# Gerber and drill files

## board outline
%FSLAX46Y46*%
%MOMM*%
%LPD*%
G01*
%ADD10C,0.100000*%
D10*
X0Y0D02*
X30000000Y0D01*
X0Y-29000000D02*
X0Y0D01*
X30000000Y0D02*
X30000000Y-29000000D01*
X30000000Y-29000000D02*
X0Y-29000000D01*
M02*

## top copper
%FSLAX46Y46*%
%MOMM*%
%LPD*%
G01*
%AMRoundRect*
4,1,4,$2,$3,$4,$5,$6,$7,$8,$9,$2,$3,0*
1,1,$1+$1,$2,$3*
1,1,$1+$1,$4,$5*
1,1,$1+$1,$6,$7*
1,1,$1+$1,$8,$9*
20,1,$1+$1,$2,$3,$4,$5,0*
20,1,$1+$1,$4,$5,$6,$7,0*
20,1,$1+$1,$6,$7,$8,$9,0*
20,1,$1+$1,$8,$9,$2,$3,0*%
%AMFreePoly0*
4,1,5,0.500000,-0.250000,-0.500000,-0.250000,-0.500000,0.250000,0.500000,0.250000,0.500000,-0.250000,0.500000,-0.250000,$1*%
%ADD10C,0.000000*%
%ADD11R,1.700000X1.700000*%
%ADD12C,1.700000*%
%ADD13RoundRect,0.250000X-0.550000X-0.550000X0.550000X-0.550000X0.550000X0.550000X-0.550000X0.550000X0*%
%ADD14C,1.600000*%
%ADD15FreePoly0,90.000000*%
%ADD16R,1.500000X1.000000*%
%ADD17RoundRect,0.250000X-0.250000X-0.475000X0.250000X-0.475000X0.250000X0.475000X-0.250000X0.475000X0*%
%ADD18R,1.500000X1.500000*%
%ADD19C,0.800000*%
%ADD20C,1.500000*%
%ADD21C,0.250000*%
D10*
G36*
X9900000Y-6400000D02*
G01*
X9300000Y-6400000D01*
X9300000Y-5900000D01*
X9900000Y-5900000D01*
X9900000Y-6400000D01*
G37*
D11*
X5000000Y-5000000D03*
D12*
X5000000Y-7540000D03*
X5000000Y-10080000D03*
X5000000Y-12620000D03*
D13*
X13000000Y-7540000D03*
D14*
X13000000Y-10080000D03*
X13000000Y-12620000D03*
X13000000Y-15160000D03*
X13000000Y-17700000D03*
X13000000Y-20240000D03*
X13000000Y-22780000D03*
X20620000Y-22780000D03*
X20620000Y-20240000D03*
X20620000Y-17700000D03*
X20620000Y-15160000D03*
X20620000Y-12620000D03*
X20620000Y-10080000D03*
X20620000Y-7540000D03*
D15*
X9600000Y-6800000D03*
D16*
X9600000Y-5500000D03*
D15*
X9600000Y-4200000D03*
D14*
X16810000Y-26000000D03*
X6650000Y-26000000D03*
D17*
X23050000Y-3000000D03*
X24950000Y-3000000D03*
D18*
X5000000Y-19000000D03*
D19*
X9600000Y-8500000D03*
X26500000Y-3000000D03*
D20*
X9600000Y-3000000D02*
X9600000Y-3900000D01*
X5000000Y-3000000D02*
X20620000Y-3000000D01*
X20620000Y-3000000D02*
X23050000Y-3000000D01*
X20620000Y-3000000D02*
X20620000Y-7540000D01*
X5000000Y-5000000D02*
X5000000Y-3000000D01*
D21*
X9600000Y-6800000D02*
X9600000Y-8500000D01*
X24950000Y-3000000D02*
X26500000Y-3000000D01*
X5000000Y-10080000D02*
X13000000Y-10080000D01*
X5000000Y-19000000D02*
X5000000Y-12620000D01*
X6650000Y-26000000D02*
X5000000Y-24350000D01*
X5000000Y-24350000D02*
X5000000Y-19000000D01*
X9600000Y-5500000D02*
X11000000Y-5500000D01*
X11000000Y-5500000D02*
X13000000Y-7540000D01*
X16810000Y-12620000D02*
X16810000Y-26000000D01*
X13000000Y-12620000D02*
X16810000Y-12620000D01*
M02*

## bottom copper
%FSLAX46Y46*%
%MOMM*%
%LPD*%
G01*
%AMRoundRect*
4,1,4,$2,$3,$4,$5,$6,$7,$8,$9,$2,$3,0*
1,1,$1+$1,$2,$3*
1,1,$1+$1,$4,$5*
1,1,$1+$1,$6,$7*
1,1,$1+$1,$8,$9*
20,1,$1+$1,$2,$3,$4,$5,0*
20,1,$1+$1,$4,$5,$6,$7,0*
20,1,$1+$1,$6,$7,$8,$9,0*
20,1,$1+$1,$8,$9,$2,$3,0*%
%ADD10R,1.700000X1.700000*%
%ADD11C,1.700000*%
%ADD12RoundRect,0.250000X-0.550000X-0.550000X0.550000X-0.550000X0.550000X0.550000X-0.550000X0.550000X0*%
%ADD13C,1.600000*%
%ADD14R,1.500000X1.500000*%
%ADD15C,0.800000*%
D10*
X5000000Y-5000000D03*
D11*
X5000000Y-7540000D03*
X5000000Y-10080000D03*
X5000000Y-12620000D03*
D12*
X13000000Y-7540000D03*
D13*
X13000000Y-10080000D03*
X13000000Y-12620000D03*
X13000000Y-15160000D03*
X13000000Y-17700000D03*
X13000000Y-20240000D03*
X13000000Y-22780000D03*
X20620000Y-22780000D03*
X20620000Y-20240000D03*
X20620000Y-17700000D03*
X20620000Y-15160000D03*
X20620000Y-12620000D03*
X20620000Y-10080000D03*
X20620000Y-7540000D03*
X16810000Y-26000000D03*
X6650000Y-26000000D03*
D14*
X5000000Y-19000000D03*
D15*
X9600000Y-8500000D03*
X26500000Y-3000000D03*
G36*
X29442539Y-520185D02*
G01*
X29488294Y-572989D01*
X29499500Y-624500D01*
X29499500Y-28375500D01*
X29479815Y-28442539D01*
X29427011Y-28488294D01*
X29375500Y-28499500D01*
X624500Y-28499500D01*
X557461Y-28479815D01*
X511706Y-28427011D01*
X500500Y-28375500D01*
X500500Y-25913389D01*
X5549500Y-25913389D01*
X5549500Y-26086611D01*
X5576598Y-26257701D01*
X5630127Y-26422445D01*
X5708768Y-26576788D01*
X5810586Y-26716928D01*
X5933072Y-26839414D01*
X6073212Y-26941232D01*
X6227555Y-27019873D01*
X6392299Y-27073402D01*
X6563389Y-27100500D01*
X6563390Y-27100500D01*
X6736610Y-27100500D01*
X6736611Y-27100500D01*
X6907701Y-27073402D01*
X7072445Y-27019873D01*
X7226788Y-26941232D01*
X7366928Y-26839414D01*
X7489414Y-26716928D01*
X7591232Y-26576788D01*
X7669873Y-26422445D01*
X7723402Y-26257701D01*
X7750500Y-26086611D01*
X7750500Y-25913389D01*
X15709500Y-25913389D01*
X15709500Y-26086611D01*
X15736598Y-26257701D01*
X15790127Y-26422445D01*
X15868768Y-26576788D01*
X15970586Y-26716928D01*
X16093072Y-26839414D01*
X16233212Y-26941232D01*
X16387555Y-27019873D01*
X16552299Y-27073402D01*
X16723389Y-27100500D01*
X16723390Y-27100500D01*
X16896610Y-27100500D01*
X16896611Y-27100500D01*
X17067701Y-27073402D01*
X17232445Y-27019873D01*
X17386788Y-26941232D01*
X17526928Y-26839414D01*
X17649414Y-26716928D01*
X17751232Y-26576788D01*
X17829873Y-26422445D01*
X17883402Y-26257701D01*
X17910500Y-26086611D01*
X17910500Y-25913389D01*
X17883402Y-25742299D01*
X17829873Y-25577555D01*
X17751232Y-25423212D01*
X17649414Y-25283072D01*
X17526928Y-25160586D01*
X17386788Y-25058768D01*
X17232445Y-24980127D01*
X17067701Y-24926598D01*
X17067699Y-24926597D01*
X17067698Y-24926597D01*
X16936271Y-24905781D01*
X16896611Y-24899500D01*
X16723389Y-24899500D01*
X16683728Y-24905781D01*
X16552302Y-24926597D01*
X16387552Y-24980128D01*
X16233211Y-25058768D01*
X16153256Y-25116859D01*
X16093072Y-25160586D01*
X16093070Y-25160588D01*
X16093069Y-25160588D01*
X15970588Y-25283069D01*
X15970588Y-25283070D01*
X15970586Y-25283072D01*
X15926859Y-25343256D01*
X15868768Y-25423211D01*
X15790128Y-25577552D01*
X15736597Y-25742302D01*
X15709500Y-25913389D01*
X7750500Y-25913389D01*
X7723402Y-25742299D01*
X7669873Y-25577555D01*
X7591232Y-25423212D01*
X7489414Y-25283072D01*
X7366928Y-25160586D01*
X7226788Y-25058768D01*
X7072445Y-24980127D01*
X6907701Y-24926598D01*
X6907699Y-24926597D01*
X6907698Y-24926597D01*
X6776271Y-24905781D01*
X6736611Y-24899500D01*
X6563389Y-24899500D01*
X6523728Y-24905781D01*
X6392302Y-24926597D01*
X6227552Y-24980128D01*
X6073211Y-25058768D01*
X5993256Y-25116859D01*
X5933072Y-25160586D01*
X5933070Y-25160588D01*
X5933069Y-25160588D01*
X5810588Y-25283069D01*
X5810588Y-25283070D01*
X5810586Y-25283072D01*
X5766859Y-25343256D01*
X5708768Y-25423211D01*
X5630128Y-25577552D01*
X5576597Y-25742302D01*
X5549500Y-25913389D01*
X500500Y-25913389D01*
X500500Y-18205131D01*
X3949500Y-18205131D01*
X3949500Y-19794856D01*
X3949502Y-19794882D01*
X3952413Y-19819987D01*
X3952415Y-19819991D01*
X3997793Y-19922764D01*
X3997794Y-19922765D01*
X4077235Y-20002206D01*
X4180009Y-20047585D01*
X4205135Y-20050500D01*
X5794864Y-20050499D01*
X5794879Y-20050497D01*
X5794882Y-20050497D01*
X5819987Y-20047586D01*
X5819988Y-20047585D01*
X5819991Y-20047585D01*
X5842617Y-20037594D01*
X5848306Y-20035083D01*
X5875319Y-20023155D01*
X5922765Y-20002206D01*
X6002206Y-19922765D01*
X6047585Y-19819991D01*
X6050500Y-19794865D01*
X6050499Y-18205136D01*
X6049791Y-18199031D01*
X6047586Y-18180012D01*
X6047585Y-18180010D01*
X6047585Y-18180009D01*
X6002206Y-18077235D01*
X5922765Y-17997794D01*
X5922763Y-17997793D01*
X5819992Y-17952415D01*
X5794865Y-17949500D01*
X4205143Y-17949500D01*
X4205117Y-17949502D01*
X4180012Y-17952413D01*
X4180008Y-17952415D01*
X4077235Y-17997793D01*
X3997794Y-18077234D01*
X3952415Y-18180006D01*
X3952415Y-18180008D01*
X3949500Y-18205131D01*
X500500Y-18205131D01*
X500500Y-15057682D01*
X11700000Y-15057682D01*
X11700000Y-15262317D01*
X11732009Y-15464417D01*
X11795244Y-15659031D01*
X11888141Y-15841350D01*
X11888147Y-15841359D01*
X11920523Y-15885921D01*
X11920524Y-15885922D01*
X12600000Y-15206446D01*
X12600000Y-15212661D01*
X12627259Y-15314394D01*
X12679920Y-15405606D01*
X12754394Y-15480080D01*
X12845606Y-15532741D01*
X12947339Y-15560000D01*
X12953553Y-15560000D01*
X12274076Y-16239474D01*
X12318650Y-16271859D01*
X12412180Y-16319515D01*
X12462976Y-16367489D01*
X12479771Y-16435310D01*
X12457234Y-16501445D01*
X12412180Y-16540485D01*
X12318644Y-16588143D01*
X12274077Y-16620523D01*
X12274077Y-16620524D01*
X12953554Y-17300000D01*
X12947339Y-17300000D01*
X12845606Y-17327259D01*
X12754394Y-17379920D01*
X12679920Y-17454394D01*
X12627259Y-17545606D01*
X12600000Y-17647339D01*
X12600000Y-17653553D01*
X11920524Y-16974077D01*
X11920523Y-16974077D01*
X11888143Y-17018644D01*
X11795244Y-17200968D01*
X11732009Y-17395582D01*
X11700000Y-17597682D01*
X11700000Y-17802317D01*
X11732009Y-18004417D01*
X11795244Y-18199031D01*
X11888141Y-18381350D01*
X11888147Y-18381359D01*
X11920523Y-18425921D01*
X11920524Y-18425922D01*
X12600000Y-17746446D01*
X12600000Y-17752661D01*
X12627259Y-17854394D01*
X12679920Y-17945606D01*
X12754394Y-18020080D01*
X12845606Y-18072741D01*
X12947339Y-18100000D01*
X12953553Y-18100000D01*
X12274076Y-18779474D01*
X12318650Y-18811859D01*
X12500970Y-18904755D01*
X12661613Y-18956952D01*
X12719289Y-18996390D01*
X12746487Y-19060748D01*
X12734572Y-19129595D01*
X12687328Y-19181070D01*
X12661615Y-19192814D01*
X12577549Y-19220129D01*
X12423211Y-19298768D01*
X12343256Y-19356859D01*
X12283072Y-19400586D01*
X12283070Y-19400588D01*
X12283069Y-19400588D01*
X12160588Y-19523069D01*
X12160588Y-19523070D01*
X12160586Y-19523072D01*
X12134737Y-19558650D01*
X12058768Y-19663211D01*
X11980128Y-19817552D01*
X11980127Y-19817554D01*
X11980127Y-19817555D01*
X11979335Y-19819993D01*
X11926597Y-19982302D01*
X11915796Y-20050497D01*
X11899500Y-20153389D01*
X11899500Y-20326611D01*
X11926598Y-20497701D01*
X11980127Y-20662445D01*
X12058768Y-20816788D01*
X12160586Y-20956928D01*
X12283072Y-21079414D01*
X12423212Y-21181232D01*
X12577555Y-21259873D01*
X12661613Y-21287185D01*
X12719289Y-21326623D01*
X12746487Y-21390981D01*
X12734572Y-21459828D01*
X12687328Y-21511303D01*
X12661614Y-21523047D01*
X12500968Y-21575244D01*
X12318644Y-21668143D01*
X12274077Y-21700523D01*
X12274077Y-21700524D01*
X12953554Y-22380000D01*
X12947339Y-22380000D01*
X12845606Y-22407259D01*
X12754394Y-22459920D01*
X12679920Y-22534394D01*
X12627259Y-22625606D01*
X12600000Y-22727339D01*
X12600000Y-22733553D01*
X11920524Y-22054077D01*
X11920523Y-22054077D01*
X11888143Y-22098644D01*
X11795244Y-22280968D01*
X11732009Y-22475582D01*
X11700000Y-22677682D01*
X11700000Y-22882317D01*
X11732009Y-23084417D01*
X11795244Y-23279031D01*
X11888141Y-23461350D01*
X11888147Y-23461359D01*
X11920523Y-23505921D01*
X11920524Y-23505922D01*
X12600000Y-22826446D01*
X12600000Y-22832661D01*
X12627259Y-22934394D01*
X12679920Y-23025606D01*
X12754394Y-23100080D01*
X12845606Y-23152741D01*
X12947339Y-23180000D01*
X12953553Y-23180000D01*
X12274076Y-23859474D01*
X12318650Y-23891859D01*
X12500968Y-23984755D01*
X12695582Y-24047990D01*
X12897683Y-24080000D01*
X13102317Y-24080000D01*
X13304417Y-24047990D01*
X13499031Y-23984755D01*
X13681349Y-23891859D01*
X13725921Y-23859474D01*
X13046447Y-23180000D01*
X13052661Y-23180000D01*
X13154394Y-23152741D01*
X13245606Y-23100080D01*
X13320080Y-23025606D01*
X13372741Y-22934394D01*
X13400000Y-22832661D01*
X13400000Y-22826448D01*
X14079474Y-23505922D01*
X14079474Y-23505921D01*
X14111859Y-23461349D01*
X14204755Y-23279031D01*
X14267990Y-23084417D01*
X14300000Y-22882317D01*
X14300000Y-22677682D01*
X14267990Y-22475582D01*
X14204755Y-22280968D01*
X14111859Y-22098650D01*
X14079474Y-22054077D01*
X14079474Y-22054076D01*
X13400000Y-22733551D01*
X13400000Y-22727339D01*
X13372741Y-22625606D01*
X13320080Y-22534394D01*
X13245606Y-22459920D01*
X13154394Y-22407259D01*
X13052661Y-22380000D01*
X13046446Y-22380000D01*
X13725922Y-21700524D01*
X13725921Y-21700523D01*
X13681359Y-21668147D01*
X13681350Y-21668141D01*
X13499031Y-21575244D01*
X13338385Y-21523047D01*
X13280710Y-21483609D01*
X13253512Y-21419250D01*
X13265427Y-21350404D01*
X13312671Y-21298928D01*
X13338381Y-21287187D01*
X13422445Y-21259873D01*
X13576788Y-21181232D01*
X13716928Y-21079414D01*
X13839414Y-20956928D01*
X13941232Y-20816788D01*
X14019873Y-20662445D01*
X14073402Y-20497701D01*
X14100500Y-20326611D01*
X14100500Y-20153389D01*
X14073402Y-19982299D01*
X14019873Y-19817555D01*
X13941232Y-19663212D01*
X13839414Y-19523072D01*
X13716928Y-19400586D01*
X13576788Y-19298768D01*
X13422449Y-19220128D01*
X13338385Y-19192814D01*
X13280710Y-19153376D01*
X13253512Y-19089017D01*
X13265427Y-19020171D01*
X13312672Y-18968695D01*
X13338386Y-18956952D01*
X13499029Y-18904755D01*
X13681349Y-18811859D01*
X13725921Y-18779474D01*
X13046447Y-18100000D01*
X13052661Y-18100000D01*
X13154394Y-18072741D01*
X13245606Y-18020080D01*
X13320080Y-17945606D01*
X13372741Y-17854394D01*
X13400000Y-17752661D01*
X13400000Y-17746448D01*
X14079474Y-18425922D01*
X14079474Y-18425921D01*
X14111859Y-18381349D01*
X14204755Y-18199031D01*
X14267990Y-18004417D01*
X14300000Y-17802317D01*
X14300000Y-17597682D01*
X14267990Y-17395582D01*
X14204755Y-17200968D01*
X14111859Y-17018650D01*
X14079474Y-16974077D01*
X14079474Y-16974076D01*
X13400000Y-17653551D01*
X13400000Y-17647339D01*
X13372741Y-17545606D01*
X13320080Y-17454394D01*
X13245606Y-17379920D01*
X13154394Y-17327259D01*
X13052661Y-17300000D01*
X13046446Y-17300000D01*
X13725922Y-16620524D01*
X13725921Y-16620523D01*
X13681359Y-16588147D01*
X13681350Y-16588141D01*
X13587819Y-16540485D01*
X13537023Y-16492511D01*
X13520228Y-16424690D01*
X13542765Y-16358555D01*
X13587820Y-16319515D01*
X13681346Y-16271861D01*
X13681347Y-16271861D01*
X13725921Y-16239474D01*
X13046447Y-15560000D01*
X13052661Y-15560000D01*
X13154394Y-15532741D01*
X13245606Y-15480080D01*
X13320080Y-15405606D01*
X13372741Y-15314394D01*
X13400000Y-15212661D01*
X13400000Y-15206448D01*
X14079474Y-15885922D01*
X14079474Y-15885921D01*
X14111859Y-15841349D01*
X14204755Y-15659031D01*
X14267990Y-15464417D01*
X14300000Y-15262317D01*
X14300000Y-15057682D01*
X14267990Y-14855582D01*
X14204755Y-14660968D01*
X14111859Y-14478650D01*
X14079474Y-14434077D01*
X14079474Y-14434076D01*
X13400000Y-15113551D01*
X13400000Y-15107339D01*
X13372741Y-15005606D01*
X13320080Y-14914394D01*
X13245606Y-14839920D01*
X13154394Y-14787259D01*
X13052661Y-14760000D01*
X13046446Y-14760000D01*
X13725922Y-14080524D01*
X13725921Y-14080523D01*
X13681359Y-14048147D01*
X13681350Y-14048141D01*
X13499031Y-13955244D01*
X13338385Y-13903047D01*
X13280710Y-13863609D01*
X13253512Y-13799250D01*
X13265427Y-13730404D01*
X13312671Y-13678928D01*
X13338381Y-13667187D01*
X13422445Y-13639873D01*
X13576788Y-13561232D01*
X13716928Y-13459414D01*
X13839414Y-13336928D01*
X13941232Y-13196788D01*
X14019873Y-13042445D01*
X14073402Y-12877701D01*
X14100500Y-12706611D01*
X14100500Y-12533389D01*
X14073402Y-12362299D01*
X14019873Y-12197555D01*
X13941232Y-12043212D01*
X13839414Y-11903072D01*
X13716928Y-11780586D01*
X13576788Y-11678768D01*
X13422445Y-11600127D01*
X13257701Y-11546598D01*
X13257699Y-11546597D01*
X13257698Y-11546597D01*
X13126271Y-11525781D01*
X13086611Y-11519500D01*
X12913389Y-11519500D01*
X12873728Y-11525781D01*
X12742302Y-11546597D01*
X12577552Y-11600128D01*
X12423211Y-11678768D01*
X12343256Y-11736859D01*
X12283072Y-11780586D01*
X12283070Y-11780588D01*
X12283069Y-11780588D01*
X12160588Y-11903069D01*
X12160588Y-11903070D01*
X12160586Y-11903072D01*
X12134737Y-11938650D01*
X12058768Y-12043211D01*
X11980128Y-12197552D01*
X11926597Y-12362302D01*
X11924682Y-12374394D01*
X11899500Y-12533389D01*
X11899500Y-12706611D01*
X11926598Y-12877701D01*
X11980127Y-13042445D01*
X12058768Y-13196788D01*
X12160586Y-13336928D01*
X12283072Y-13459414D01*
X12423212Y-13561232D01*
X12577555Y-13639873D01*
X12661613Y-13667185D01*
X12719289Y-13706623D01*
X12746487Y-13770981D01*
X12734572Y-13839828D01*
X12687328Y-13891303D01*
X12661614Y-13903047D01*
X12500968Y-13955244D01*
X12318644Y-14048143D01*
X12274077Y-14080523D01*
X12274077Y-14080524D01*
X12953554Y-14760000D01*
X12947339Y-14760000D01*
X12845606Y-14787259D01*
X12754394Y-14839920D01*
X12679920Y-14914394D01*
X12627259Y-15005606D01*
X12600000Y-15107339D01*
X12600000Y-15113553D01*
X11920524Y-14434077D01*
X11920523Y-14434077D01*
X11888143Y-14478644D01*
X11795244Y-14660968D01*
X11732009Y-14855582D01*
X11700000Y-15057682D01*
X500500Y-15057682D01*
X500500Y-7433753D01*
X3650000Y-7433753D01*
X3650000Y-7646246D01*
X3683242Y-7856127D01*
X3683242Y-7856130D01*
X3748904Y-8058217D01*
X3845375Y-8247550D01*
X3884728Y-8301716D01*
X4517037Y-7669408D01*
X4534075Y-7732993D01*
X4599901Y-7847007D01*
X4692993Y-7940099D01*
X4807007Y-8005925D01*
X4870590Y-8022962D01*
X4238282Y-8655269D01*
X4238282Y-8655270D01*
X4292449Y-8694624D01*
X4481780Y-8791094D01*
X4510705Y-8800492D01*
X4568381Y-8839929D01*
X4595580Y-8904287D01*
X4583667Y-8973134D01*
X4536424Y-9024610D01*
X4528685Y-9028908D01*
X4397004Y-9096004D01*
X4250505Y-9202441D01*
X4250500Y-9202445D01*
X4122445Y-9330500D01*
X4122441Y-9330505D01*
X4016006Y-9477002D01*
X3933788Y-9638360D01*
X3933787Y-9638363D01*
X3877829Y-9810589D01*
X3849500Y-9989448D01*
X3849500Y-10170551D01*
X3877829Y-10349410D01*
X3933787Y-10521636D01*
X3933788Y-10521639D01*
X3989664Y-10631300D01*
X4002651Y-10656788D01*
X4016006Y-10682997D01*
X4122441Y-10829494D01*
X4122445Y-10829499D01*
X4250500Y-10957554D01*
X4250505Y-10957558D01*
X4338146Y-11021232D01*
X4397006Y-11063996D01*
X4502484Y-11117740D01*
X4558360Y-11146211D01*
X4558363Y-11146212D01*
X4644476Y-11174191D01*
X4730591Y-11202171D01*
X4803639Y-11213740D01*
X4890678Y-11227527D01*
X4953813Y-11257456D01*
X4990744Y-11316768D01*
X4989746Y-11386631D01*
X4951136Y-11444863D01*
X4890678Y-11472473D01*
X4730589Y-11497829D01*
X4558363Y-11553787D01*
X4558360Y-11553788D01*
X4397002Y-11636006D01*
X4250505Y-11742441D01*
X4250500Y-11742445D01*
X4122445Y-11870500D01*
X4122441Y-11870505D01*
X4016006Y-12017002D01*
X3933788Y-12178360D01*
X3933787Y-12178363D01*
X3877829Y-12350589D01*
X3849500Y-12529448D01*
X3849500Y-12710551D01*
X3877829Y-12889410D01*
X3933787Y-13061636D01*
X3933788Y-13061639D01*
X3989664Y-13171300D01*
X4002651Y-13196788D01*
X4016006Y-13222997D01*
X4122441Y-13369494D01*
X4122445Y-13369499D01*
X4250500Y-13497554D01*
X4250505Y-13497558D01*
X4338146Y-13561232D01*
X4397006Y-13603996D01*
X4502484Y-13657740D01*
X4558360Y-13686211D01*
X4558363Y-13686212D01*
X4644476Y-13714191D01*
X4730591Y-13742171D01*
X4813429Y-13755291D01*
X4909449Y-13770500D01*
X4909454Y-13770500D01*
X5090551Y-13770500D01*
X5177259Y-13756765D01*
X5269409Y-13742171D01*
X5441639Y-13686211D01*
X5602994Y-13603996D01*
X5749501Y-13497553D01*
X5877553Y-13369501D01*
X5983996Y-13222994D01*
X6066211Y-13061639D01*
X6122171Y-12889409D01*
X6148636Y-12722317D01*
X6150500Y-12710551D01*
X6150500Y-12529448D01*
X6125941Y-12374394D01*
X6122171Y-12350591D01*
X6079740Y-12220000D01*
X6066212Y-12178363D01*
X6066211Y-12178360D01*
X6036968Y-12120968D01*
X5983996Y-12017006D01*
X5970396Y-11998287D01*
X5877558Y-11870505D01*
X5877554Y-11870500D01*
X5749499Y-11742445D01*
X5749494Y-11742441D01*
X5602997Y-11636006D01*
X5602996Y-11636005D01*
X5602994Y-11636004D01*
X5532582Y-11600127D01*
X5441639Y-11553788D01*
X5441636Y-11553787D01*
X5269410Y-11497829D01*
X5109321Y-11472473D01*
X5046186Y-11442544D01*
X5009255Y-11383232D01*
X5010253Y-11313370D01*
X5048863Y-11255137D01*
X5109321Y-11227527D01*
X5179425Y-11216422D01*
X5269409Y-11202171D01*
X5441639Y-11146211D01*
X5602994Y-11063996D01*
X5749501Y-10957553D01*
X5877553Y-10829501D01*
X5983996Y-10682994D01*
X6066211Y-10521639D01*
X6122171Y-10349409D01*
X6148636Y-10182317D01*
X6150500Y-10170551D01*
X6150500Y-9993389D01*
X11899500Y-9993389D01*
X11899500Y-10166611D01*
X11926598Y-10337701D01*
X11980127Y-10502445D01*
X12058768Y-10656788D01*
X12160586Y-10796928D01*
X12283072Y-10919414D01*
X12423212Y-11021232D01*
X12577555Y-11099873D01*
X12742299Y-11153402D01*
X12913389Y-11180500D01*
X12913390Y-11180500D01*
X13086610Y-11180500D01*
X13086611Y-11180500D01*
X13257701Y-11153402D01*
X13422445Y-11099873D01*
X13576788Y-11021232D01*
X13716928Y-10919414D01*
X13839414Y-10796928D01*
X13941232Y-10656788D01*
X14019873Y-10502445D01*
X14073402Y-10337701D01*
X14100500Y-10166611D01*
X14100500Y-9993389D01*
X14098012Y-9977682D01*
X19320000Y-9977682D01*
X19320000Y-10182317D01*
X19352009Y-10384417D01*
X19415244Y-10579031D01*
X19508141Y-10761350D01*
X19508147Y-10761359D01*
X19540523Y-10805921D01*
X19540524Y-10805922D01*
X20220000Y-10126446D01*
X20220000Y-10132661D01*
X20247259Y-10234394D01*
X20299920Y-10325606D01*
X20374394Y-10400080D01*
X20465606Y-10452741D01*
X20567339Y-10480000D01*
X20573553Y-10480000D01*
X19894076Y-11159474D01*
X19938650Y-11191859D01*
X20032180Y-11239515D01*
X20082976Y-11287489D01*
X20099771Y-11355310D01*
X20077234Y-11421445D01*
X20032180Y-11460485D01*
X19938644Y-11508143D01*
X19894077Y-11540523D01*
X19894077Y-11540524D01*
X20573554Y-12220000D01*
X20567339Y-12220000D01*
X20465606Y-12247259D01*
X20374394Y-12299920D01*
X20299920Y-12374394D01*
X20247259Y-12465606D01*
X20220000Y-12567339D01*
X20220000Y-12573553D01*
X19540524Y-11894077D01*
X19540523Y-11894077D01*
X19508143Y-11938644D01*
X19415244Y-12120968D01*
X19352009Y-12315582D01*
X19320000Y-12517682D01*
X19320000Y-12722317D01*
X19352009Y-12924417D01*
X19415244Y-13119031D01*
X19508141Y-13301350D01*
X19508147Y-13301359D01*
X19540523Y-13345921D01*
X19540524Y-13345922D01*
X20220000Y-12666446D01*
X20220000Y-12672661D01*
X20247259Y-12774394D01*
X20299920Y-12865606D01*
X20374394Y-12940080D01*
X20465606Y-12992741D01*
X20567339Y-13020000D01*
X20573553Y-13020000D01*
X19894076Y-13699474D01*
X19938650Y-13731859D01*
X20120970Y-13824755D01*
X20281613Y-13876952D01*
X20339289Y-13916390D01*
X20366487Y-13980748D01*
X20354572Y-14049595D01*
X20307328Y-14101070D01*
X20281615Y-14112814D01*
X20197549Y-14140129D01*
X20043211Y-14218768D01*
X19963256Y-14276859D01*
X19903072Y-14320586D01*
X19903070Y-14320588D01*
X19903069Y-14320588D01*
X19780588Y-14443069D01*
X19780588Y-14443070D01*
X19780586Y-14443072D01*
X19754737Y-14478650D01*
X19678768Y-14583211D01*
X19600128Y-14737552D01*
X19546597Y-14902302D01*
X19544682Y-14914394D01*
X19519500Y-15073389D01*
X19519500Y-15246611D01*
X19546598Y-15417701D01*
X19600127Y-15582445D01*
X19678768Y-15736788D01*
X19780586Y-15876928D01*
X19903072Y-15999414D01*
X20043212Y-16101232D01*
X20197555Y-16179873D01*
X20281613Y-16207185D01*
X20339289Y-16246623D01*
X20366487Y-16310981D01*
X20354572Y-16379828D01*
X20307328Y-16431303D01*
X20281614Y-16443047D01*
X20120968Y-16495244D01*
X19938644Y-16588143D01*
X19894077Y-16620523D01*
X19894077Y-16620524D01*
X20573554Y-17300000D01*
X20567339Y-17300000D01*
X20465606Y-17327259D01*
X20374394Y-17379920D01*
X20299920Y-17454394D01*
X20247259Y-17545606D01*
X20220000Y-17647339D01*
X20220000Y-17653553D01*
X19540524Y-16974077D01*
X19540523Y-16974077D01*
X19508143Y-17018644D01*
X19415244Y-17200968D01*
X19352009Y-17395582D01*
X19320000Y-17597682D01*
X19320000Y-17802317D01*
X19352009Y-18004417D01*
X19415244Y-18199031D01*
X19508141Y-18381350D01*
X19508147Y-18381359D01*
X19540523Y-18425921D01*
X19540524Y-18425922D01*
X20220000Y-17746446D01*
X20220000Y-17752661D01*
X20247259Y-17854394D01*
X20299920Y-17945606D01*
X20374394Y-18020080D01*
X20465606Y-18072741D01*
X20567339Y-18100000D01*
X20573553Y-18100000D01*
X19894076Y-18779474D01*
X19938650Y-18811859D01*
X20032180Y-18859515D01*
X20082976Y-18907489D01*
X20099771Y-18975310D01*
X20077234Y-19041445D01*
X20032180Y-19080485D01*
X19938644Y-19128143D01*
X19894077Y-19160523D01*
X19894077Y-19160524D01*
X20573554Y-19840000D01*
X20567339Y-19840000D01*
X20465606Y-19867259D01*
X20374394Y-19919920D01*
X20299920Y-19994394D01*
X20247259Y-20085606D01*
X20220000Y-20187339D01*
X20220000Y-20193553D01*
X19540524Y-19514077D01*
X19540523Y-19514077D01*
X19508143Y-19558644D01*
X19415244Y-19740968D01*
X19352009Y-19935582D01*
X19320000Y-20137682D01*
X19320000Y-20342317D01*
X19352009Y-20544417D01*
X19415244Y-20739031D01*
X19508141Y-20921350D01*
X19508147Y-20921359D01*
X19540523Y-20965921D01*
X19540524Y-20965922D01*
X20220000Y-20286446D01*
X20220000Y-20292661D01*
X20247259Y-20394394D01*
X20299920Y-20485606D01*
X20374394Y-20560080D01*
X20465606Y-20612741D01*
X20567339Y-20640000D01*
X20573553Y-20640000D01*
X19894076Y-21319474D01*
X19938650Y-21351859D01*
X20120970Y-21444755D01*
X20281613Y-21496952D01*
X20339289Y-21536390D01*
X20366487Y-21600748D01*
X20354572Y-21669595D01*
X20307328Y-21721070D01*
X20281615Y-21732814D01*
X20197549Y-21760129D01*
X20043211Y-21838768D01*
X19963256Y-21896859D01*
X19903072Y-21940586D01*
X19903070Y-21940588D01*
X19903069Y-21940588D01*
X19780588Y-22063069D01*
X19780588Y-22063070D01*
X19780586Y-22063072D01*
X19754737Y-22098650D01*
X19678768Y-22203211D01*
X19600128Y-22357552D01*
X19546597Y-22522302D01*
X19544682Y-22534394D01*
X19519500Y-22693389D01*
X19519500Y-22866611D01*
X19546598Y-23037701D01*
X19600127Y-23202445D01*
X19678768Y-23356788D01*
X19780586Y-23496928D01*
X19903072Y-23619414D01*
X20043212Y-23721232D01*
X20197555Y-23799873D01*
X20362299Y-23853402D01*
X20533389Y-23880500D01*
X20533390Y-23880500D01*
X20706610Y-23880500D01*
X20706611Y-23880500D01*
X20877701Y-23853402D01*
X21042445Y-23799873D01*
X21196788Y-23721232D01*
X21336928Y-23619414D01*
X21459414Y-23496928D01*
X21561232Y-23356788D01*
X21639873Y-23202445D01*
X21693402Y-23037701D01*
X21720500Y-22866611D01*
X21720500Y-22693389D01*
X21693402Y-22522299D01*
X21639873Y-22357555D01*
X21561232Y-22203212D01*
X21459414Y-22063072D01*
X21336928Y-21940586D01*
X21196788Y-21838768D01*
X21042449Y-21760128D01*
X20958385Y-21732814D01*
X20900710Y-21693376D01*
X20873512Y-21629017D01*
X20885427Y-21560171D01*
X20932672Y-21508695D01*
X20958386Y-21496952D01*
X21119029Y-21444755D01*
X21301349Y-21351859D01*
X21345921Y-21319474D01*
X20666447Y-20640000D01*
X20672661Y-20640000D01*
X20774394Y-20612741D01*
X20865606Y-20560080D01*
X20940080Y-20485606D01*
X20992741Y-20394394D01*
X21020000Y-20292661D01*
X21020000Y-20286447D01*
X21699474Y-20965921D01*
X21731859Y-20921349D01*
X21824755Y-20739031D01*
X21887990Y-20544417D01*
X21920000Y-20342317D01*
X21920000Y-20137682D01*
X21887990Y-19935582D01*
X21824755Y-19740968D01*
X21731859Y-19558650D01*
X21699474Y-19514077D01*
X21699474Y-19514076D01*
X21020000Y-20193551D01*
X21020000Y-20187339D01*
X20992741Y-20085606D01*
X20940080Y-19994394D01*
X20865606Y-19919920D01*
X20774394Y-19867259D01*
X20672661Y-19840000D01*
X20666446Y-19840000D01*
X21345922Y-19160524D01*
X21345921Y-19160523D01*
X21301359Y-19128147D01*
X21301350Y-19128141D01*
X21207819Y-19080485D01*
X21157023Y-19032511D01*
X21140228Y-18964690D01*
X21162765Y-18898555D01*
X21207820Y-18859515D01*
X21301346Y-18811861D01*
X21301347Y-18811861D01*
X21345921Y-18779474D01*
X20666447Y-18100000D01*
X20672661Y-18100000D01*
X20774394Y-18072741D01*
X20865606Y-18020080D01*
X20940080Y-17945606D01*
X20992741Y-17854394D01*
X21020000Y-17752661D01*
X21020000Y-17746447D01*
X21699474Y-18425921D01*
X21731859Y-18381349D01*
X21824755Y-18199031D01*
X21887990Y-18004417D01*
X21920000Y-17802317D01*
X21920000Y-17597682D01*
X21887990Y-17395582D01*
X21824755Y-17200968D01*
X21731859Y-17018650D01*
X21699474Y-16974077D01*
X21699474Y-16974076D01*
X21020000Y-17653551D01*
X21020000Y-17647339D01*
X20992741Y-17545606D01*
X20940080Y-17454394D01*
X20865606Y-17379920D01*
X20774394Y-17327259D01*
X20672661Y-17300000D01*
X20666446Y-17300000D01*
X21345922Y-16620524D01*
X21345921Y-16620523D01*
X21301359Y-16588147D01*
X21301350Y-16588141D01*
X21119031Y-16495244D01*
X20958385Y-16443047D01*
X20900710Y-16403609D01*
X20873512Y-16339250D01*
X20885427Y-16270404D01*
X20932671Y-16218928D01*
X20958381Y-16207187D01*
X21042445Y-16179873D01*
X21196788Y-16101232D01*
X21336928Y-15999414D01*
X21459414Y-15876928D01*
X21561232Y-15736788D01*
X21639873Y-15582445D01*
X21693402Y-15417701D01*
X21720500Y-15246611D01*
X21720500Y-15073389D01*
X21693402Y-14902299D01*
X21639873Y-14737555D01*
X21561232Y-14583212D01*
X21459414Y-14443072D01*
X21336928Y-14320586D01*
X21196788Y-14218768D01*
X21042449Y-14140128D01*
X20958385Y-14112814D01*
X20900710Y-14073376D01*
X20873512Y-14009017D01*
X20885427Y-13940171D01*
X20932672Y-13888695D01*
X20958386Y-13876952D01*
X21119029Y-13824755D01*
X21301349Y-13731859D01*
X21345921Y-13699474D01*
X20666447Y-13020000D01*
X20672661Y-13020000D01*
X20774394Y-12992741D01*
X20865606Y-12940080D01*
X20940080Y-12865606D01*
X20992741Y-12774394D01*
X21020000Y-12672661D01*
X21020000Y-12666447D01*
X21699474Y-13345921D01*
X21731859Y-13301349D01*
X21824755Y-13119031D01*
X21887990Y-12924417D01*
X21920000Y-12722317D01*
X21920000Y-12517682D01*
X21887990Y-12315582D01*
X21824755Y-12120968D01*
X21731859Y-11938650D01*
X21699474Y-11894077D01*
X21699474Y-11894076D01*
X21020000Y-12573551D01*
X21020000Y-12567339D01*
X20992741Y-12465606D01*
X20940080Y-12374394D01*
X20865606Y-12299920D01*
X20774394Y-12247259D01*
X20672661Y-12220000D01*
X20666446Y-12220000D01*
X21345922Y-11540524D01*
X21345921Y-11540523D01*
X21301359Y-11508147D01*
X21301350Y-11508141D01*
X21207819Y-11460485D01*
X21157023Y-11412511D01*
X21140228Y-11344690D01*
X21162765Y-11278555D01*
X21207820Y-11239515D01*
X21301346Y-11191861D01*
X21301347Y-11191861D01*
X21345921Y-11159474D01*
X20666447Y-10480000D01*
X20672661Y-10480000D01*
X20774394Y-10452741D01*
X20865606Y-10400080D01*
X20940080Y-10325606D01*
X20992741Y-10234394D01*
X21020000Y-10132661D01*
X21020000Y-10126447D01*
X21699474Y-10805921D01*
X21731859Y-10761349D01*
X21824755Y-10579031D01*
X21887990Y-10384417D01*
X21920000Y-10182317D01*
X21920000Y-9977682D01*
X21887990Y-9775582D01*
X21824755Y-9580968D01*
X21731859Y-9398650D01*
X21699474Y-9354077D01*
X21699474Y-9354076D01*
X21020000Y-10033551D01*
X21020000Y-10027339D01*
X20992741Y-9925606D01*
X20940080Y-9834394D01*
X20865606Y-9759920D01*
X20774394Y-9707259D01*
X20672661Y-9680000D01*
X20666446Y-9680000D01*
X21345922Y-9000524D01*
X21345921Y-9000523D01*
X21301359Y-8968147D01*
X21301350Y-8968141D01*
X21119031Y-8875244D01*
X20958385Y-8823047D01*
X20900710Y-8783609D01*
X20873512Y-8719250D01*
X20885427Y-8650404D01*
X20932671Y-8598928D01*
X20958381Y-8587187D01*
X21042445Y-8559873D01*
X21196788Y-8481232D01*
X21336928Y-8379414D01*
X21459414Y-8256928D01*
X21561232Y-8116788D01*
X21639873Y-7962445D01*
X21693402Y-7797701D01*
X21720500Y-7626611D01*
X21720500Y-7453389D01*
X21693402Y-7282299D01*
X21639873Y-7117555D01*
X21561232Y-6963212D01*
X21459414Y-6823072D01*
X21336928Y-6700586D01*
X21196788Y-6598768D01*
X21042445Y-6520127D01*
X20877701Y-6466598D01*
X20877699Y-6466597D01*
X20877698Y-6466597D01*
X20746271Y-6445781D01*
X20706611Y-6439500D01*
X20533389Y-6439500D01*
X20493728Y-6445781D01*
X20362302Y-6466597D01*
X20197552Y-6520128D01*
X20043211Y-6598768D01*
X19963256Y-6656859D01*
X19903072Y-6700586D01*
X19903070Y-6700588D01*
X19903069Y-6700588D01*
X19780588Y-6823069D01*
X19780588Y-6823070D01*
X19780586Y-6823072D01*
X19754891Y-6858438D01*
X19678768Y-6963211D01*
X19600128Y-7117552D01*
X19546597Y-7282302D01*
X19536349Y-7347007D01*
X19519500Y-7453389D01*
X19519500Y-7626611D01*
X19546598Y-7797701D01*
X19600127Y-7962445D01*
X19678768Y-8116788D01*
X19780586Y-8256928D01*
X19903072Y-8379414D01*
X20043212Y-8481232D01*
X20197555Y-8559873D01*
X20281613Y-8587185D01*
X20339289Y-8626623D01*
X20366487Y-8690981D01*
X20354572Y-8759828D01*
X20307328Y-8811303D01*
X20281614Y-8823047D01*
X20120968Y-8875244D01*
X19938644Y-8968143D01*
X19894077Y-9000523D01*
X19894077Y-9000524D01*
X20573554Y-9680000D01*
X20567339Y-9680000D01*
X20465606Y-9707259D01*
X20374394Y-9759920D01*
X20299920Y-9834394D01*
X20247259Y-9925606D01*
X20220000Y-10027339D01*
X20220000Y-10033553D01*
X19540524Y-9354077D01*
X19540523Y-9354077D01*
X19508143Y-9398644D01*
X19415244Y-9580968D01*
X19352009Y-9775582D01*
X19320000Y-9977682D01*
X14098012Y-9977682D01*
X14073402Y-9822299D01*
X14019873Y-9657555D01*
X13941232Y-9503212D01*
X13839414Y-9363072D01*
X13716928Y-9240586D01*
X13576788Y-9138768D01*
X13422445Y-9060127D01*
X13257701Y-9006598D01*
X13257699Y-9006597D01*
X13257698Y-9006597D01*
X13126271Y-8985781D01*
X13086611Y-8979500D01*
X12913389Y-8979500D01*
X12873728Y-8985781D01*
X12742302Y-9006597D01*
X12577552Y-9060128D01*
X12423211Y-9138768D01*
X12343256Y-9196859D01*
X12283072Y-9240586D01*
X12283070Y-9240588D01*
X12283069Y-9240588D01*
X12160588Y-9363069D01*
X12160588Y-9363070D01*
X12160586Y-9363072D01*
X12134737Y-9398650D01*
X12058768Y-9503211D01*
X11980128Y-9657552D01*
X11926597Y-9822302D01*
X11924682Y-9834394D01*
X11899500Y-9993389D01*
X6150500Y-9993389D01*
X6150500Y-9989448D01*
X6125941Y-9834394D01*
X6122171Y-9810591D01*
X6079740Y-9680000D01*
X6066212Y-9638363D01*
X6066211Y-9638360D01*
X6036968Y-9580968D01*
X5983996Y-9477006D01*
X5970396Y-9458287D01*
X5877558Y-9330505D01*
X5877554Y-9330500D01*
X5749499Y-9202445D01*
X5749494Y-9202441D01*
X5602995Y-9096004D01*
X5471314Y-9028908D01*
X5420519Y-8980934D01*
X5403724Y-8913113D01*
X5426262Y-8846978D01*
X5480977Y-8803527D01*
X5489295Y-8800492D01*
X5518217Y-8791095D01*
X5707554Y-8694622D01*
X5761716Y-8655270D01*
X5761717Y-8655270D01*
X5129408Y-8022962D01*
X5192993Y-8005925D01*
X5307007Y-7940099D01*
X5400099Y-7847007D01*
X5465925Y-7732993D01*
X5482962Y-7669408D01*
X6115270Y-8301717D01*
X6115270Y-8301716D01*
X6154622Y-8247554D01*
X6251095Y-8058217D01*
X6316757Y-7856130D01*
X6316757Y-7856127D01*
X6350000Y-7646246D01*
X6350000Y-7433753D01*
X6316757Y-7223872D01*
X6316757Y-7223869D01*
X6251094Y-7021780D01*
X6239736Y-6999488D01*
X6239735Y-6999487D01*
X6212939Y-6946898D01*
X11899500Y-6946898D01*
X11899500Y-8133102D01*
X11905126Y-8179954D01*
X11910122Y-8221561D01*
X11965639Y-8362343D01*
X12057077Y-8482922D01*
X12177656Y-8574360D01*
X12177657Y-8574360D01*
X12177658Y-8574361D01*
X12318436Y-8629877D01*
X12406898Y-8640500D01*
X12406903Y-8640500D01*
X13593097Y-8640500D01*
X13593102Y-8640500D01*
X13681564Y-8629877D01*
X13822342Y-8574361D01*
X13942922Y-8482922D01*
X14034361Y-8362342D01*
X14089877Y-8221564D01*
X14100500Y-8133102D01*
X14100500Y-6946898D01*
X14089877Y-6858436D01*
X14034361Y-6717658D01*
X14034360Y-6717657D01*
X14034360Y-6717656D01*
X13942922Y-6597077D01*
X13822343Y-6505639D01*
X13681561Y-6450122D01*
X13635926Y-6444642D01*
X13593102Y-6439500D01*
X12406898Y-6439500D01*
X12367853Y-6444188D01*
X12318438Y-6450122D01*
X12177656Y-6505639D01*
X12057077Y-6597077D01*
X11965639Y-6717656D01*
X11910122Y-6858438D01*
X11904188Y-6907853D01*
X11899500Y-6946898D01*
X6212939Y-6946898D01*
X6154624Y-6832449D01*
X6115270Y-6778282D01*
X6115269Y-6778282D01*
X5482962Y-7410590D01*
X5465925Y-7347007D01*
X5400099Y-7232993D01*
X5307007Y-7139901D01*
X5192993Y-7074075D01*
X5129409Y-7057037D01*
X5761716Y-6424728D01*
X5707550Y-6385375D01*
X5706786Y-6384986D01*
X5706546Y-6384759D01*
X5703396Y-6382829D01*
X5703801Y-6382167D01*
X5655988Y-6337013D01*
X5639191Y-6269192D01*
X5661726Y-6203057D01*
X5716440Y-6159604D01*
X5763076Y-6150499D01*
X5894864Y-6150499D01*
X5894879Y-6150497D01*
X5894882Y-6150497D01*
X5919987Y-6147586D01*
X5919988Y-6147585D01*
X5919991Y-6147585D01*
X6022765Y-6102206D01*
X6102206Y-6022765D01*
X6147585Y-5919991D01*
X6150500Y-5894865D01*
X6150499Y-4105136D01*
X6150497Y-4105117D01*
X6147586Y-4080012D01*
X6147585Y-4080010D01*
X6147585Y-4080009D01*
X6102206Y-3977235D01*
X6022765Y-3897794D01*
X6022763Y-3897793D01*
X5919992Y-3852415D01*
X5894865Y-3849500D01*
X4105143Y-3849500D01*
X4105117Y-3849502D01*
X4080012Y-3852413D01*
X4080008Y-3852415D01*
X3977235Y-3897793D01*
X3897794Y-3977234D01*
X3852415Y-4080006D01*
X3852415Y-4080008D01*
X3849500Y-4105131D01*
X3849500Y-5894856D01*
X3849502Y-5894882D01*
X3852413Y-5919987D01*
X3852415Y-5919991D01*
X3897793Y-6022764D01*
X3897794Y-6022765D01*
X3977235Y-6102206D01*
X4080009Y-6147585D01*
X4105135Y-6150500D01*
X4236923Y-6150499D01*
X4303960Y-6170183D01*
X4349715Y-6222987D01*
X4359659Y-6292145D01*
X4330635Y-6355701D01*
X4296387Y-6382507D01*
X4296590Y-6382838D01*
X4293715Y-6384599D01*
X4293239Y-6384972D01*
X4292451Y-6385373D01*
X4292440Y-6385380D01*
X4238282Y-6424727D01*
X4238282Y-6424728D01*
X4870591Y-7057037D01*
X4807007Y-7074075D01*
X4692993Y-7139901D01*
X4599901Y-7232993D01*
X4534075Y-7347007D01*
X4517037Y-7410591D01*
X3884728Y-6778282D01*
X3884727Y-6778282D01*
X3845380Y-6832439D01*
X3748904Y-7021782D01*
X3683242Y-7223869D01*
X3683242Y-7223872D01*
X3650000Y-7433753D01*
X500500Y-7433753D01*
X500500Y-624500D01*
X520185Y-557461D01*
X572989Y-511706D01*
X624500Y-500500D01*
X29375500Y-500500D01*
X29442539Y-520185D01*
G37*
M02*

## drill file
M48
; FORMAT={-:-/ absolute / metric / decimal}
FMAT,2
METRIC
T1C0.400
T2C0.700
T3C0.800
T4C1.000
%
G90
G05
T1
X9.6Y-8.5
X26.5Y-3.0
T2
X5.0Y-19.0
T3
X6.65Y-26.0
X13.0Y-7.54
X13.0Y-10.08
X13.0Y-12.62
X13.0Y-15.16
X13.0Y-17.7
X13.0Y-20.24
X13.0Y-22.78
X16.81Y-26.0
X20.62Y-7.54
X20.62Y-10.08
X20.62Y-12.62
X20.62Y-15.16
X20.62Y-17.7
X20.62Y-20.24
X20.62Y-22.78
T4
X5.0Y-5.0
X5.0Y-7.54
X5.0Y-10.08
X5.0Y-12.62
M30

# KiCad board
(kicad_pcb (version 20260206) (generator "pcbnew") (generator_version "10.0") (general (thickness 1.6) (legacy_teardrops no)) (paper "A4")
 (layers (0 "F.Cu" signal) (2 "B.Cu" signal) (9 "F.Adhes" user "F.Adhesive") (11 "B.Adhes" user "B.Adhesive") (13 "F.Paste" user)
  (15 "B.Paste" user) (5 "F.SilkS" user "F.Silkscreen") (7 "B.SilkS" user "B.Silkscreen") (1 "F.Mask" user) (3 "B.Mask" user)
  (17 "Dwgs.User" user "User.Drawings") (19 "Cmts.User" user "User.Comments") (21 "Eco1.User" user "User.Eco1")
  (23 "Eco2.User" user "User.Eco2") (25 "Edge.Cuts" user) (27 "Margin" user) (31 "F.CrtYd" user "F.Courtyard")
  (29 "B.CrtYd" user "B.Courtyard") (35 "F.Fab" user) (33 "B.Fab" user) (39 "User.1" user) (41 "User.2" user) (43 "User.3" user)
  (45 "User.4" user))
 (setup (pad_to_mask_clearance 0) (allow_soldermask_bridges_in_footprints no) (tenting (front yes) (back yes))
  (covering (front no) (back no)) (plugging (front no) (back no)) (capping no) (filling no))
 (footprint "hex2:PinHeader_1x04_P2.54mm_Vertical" (layer "F.Cu") (at 5 5)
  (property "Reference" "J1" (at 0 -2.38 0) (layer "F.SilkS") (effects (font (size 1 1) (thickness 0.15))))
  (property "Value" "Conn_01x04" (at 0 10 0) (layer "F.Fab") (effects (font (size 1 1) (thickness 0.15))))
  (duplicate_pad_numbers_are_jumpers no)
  (pad "1" thru_hole rect (at 0 0) (size 1.7 1.7) (drill 1) (layers "*.Cu" "*.Mask") (remove_unused_layers no) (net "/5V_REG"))
  (pad "2" thru_hole circle (at 0 2.54) (size 1.7 1.7) (drill 1) (layers "*.Cu" "*.Mask") (remove_unused_layers no) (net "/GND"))
  (pad "3" thru_hole circle (at 0 5.08) (size 1.7 1.7) (drill 1) (layers "*.Cu" "*.Mask") (remove_unused_layers no) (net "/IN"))
  (pad "4" thru_hole circle (at 0 7.62) (size 1.7 1.7) (drill 1) (layers "*.Cu" "*.Mask") (remove_unused_layers no) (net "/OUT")))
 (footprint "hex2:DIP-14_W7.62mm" (layer "F.Cu") (at 13 7.54)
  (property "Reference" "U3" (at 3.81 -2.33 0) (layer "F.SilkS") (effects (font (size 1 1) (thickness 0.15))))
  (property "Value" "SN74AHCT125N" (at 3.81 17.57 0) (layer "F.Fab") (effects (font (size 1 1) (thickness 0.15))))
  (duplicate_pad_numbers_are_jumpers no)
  (pad "1" thru_hole roundrect (at 0 0) (size 1.6 1.6) (drill 0.8) (layers "*.Cu" "*.Mask") (remove_unused_layers no)
   (roundrect_rratio 0.15625) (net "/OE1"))
  (pad "2" thru_hole circle (at 0 2.54) (size 1.6 1.6) (drill 0.8) (layers "*.Cu" "*.Mask") (remove_unused_layers no) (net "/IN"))
  (pad "3" thru_hole circle (at 0 5.08) (size 1.6 1.6) (drill 0.8) (layers "*.Cu" "*.Mask") (remove_unused_layers no) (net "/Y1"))
  (pad "4" thru_hole circle (at 0 7.62) (size 1.6 1.6) (drill 0.8) (layers "*.Cu" "*.Mask") (remove_unused_layers no) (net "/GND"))
  (pad "5" thru_hole circle (at 0 10.16) (size 1.6 1.6) (drill 0.8) (layers "*.Cu" "*.Mask") (remove_unused_layers no) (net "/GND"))
  (pad "6" thru_hole circle (at 0 12.7) (size 1.6 1.6) (drill 0.8) (layers "*.Cu" "*.Mask") (remove_unused_layers no)
   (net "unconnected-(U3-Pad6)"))
  (pad "7" thru_hole circle (at 0 15.24) (size 1.6 1.6) (drill 0.8) (layers "*.Cu" "*.Mask") (remove_unused_layers no) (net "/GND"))
  (pad "8" thru_hole circle (at 7.62 15.24) (size 1.6 1.6) (drill 0.8) (layers "*.Cu" "*.Mask") (remove_unused_layers no)
   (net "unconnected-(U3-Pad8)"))
  (pad "9" thru_hole circle (at 7.62 12.7) (size 1.6 1.6) (drill 0.8) (layers "*.Cu" "*.Mask") (remove_unused_layers no) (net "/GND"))
  (pad "10" thru_hole circle (at 7.62 10.16) (size 1.6 1.6) (drill 0.8) (layers "*.Cu" "*.Mask") (remove_unused_layers no) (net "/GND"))
  (pad "11" thru_hole circle (at 7.62 7.62) (size 1.6 1.6) (drill 0.8) (layers "*.Cu" "*.Mask") (remove_unused_layers no)
   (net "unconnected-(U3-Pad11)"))
  (pad "12" thru_hole circle (at 7.62 5.08) (size 1.6 1.6) (drill 0.8) (layers "*.Cu" "*.Mask") (remove_unused_layers no) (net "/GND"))
  (pad "13" thru_hole circle (at 7.62 2.54) (size 1.6 1.6) (drill 0.8) (layers "*.Cu" "*.Mask") (remove_unused_layers no) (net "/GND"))
  (pad "14" thru_hole circle (at 7.62 0) (size 1.6 1.6) (drill 0.8) (layers "*.Cu" "*.Mask") (remove_unused_layers no) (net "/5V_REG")))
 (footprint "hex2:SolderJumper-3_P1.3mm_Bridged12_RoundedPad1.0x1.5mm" (layer "F.Cu") (at 9.6 5.5 90)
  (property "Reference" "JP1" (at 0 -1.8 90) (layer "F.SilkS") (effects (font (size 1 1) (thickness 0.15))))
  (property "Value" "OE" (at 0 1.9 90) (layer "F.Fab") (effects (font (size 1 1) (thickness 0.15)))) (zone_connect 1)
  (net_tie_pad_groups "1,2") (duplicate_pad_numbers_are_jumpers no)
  (fp_poly (pts (xy -0.9 -0.3) (xy -0.4 -0.3) (xy -0.4 0.3) (xy -0.9 0.3)) (stroke (width 0) (type solid)) (fill yes) (layer "F.Cu"))
  (pad "1" smd custom (at -1.3 0 90) (size 1 0.5) (layers "F.Cu" "F.Mask") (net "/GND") (zone_connect 2) (thermal_bridge_angle 45)
   (options (clearance outline) (anchor rect)) (primitives))
  (pad "2" smd rect (at 0 0 90) (size 1 1.5) (layers "F.Cu" "F.Mask") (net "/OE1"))
  (pad "3" smd custom (at 1.3 0 90) (size 1 0.5) (layers "F.Cu" "F.Mask") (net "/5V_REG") (zone_connect 2) (thermal_bridge_angle 45)
   (options (clearance outline) (anchor rect)) (primitives)))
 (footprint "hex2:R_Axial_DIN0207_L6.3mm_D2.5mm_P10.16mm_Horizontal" (layer "F.Cu") (at 16.81 26 180)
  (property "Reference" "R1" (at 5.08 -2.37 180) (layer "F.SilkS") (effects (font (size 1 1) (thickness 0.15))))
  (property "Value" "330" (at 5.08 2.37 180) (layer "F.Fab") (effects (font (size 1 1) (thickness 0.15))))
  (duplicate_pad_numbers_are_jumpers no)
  (pad "1" thru_hole circle (at 0 0 180) (size 1.6 1.6) (drill 0.8) (layers "*.Cu" "*.Mask") (remove_unused_layers no) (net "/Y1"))
  (pad "2" thru_hole circle (at 10.16 0 180) (size 1.6 1.6) (drill 0.8) (layers "*.Cu" "*.Mask") (remove_unused_layers no) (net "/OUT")))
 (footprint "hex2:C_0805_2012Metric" (layer "F.Cu") (at 24 3)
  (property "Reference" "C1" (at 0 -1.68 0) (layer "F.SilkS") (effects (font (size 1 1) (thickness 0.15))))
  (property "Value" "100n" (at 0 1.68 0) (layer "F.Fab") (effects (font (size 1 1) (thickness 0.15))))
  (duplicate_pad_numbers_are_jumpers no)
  (pad "1" smd roundrect (at -0.95 0) (size 1 1.45) (layers "F.Cu" "F.Mask" "F.Paste") (roundrect_rratio 0.25) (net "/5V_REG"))
  (pad "2" smd roundrect (at 0.95 0) (size 1 1.45) (layers "F.Cu" "F.Mask" "F.Paste") (roundrect_rratio 0.25) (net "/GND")))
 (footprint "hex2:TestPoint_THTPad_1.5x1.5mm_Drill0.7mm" (layer "F.Cu") (at 5 19)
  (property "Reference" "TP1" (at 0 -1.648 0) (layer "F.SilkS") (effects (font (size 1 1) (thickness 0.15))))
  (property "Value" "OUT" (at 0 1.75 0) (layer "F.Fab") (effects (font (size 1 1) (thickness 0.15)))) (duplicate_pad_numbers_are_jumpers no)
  (pad "1" thru_hole rect (at 0 0) (size 1.5 1.5) (drill 0.7) (layers "*.Cu" "*.Mask") (remove_unused_layers no) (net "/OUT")))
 (gr_line (start 0 0) (end 30 0) (stroke (width 0.1) (type default)) (layer "Edge.Cuts"))
 (gr_line (start 0 29) (end 0 0) (stroke (width 0.1) (type default)) (layer "Edge.Cuts"))
 (gr_line (start 30 0) (end 30 29) (stroke (width 0.1) (type default)) (layer "Edge.Cuts"))
 (gr_line (start 30 29) (end 0 29) (stroke (width 0.1) (type default)) (layer "Edge.Cuts"))
 (segment (start 9.6 3) (end 9.6 3.9) (width 1.5) (layer "F.Cu") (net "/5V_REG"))
 (segment (start 5 3) (end 20.62 3) (width 1.5) (layer "F.Cu") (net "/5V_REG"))
 (segment (start 20.62 3) (end 23.05 3) (width 1.5) (layer "F.Cu") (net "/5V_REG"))
 (segment (start 20.62 3) (end 20.62 7.54) (width 1.5) (layer "F.Cu") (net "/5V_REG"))
 (segment (start 5 5) (end 5 3) (width 1.5) (layer "F.Cu") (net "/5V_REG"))
 (segment (start 9.6 6.8) (end 9.6 8.5) (width 0.25) (layer "F.Cu") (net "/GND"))
 (segment (start 24.95 3) (end 26.5 3) (width 0.25) (layer "F.Cu") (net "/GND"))
 (via (at 9.6 8.5) (size 0.8) (drill 0.4) (layers "F.Cu" "B.Cu") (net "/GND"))
 (via (at 26.5 3) (size 0.8) (drill 0.4) (layers "F.Cu" "B.Cu") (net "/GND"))
 (segment (start 5 10.08) (end 13 10.08) (width 0.25) (layer "F.Cu") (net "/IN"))
 (segment (start 5 19) (end 5 12.62) (width 0.25) (layer "F.Cu") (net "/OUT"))
 (segment (start 6.65 26) (end 5 24.35) (width 0.25) (layer "F.Cu") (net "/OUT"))
 (segment (start 5 24.35) (end 5 19) (width 0.25) (layer "F.Cu") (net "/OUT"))
 (segment (start 9.6 5.5) (end 11 5.5) (width 0.25) (layer "F.Cu") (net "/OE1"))
 (segment (start 11 5.5) (end 13 7.54) (width 0.25) (layer "F.Cu") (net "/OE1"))
 (segment (start 16.81 12.62) (end 16.81 26) (width 0.25) (layer "F.Cu") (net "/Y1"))
 (segment (start 13 12.62) (end 16.81 12.62) (width 0.25) (layer "F.Cu") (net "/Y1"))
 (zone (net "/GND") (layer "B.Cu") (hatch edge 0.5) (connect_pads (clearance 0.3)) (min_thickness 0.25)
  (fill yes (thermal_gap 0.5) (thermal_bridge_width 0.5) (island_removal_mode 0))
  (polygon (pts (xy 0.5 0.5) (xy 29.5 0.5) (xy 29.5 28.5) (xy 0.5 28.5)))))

